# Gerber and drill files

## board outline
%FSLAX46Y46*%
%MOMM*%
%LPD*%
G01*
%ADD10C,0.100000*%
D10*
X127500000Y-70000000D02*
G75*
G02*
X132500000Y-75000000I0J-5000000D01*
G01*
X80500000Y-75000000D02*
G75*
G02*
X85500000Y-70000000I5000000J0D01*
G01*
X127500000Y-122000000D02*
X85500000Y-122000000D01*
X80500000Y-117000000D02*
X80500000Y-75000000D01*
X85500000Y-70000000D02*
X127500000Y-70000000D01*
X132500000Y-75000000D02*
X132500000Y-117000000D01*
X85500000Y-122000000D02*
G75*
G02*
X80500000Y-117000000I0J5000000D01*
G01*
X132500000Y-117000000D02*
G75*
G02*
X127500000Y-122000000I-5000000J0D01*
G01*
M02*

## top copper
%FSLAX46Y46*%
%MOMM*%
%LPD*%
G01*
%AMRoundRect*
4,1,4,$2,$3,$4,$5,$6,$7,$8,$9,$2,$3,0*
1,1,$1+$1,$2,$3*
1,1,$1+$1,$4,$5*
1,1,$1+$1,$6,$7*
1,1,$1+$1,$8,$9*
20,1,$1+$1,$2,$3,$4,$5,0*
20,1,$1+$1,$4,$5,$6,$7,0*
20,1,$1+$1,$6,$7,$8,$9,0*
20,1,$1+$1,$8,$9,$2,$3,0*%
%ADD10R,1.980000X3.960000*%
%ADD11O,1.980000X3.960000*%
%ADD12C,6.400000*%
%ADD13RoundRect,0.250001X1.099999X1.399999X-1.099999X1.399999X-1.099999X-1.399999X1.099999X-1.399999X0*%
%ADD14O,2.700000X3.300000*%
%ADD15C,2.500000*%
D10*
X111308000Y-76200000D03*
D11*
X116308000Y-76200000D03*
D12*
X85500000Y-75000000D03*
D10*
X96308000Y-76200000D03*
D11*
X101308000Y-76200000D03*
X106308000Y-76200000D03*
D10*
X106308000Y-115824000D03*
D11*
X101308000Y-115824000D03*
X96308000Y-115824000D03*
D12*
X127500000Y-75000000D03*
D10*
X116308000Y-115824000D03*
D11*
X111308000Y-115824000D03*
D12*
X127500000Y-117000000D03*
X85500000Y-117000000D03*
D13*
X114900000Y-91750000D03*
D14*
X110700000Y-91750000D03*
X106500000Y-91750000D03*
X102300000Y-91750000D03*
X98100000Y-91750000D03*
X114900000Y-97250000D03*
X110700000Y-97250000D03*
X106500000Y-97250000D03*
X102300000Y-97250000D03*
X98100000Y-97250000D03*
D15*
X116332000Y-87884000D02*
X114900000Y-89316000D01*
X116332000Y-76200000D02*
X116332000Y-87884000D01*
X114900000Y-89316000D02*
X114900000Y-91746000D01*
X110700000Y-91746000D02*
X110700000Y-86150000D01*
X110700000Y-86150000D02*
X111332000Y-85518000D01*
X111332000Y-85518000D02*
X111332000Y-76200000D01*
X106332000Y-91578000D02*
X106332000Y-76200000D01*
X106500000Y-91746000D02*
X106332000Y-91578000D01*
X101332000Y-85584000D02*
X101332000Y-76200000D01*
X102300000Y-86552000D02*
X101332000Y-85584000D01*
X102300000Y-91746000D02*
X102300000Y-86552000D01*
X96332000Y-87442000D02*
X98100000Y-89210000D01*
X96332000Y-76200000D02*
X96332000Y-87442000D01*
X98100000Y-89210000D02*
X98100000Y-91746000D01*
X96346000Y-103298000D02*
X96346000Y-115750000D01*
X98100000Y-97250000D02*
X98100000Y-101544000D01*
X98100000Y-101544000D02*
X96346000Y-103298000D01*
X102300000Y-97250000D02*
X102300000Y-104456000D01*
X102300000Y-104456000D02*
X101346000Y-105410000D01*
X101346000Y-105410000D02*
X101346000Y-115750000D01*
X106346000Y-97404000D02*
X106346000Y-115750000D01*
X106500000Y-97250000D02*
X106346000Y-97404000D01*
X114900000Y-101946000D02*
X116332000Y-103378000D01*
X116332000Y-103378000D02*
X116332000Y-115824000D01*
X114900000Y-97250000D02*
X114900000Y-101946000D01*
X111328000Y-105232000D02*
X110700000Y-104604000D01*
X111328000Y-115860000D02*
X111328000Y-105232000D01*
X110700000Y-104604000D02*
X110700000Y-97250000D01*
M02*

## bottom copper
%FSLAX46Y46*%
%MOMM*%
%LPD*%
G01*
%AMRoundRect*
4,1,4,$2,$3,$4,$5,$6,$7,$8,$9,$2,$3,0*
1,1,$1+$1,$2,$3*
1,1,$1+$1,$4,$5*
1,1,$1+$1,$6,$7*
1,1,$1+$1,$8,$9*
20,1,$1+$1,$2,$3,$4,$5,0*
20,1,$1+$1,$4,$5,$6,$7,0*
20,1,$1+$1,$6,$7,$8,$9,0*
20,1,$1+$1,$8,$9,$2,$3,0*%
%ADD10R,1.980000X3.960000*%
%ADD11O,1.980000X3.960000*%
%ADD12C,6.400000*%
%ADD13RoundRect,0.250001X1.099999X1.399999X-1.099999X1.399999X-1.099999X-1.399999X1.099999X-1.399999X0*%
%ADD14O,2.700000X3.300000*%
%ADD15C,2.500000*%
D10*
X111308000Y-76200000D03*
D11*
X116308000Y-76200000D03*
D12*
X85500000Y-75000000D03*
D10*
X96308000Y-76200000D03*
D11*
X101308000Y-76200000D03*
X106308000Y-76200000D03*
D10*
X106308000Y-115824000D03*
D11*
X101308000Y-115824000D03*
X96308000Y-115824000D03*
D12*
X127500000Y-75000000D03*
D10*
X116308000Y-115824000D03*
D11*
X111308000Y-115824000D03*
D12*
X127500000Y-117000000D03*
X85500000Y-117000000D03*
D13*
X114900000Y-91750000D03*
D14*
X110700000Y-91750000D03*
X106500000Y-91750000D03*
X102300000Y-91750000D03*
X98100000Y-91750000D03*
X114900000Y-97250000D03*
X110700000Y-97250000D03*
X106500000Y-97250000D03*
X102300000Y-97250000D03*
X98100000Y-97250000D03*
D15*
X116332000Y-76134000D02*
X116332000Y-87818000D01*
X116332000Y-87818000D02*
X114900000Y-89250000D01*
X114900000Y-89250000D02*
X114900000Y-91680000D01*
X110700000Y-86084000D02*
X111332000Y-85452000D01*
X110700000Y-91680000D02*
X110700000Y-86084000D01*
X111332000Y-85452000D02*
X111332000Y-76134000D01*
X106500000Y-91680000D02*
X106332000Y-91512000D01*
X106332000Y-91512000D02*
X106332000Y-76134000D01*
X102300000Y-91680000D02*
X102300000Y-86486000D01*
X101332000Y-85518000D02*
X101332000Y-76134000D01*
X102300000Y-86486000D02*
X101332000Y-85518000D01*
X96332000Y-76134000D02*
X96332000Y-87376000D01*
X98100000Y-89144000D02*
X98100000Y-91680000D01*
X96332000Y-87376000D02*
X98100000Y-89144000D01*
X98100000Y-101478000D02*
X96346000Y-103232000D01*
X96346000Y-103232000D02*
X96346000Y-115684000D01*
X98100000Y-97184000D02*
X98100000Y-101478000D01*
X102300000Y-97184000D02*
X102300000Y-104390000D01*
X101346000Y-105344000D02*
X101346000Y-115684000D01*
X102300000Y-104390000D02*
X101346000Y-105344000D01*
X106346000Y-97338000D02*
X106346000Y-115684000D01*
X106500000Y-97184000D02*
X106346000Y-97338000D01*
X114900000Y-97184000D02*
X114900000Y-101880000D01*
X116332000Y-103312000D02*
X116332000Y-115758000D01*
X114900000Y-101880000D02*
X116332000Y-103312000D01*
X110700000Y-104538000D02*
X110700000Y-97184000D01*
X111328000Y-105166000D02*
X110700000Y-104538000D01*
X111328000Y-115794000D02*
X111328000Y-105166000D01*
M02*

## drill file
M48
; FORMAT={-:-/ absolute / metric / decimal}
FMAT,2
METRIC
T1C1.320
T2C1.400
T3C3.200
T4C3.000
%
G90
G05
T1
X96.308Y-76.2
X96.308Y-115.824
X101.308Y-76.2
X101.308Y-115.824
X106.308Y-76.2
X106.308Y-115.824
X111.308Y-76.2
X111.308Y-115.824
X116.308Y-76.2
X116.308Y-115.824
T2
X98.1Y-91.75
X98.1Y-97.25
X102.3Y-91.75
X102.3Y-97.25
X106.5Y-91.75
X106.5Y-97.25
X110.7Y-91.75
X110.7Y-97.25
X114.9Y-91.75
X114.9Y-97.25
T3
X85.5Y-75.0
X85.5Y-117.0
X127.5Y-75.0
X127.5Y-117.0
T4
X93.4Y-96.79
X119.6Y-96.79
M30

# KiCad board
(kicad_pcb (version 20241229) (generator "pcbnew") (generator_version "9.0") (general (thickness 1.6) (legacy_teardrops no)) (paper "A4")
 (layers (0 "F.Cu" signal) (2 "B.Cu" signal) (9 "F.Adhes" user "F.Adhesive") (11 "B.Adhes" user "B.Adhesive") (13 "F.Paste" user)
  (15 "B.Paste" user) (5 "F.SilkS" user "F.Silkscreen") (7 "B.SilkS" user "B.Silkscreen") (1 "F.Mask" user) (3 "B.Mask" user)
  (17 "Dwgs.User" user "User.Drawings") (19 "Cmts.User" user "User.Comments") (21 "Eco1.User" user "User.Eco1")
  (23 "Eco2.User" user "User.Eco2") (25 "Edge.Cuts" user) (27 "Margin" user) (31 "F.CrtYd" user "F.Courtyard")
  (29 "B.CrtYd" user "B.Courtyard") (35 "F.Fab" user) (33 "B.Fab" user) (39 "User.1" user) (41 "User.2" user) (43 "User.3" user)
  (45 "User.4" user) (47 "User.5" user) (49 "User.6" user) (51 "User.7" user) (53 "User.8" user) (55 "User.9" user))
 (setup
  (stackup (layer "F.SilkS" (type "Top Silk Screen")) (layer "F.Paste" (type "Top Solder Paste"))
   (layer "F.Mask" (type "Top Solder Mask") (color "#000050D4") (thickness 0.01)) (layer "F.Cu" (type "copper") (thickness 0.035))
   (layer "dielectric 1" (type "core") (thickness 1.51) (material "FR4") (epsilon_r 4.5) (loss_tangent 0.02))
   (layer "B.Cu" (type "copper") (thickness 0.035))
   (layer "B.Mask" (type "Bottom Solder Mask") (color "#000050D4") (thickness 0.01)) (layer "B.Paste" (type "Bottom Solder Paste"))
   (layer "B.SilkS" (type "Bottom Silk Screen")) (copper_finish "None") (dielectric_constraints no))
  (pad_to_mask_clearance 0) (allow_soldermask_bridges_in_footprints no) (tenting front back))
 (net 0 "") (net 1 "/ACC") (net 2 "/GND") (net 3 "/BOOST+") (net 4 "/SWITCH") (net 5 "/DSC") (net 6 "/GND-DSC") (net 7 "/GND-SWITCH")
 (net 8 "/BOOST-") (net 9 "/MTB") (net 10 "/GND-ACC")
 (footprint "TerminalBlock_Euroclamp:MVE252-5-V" (layer "F.Cu") (at 113.808 76.2)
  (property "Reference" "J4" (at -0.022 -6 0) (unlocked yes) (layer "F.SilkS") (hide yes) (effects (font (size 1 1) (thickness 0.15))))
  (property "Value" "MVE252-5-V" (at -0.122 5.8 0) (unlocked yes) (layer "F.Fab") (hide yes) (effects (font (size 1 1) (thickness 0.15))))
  (pad "1" thru_hole rect (at -2.5 0) (size 1.98 3.96) (drill 1.32) (layers "*.Cu" "*.Mask") (remove_unused_layers no) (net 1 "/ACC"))
  (pad "2" thru_hole oval (at 2.5 0) (size 1.98 3.96) (drill 1.32) (layers "*.Cu" "*.Mask") (remove_unused_layers no) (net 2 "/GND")))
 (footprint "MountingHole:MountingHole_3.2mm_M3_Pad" (layer "F.Cu") (at 85.5 75)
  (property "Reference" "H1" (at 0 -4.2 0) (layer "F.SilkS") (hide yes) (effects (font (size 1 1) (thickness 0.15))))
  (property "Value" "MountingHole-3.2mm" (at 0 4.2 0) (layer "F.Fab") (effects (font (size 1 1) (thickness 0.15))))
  (pad "1" thru_hole circle (at 0 0) (size 6.4 6.4) (drill 3.2) (layers "*.Cu" "*.Mask") (remove_unused_layers no)))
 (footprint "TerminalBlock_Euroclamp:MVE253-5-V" (layer "F.Cu") (at 101.308 76.2)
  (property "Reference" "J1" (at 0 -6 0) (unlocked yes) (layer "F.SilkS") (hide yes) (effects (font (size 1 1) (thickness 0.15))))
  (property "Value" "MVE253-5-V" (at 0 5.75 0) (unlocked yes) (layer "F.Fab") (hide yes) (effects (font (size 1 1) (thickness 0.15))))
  (pad "1" thru_hole rect (at -5 0) (size 1.98 3.96) (drill 1.32) (layers "*.Cu" "*.Mask") (remove_unused_layers no) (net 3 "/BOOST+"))
  (pad "2" thru_hole oval (at 0 0) (size 1.98 3.96) (drill 1.32) (layers "*.Cu" "*.Mask") (remove_unused_layers no) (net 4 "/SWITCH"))
  (pad "3" thru_hole oval (at 5 0) (size 1.98 3.96) (drill 1.32) (layers "*.Cu" "*.Mask") (remove_unused_layers no) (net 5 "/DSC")))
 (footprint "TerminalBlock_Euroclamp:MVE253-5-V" (layer "F.Cu") (at 101.308 115.824 180)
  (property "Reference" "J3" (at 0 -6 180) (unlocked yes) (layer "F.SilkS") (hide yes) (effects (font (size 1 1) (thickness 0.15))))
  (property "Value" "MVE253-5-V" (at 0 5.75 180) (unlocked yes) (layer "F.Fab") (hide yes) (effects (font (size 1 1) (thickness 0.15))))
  (pad "1" thru_hole rect (at -5 0 180) (size 1.98 3.96) (drill 1.32) (layers "*.Cu" "*.Mask") (remove_unused_layers no) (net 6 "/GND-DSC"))
  (pad "2" thru_hole oval (at 0 0 180) (size 1.98 3.96) (drill 1.32) (layers "*.Cu" "*.Mask") (remove_unused_layers no)
   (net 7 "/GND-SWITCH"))
  (pad "3" thru_hole oval (at 5 0 180) (size 1.98 3.96) (drill 1.32) (layers "*.Cu" "*.Mask") (remove_unused_layers no) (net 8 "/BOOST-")))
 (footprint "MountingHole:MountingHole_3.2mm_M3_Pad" (layer "F.Cu") (at 127.5 75)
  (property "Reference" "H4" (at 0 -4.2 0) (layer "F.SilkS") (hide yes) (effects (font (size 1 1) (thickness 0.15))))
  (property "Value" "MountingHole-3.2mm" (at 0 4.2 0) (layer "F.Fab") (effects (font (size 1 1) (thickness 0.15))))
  (pad "1" thru_hole circle (at 0 0) (size 6.4 6.4) (drill 3.2) (layers "*.Cu" "*.Mask") (remove_unused_layers no)))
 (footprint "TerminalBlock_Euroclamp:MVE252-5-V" (layer "F.Cu") (at 113.808 115.824 180)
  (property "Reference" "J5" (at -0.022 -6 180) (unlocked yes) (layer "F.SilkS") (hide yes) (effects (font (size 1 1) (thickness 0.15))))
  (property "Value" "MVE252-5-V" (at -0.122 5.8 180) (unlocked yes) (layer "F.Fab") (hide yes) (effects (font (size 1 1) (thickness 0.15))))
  (pad "1" thru_hole rect (at -2.5 0 180) (size 1.98 3.96) (drill 1.32) (layers "*.Cu" "*.Mask") (remove_unused_layers no) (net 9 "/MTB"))
  (pad "2" thru_hole oval (at 2.5 0 180) (size 1.98 3.96) (drill 1.32) (layers "*.Cu" "*.Mask") (remove_unused_layers no)
   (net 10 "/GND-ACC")))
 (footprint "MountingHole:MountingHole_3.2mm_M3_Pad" (layer "F.Cu") (at 127.5 117)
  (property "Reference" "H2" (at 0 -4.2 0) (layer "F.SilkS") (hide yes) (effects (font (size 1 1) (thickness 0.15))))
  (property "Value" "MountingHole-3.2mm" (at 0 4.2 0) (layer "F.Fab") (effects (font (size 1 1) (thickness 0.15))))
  (pad "1" thru_hole circle (at 0 0) (size 6.4 6.4) (drill 3.2) (layers "*.Cu" "*.Mask") (remove_unused_layers no)))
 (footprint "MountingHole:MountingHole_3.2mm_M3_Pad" (layer "F.Cu") (at 85.5 117)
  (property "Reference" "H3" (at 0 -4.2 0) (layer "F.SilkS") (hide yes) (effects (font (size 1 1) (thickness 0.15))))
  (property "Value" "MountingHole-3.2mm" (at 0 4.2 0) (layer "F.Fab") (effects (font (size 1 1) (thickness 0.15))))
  (pad "1" thru_hole circle (at 0 0) (size 6.4 6.4) (drill 3.2) (layers "*.Cu" "*.Mask") (remove_unused_layers no)))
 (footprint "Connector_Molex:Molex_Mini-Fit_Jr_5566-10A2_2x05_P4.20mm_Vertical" (layer "B.Cu") (at 114.9 91.75 180)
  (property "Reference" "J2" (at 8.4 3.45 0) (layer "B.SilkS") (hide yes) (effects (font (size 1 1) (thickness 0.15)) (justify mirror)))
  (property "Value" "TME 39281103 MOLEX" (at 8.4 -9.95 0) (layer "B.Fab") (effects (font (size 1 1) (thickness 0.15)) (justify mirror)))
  (pad "" np_thru_hole circle (at -4.7 -5.04 180) (size 3 3) (drill 3) (layers "*.Cu" "*.Mask"))
  (pad "" np_thru_hole circle (at 21.5 -5.04 180) (size 3 3) (drill 3) (layers "*.Cu" "*.Mask"))
  (pad "1" thru_hole roundrect (at 0 0 180) (size 2.7 3.3) (drill 1.4) (layers "*.Cu" "*.Mask") (remove_unused_layers no)
   (roundrect_rratio 0.092593) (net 2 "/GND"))
  (pad "2" thru_hole oval (at 4.2 0 180) (size 2.7 3.3) (drill 1.4) (layers "*.Cu" "*.Mask") (remove_unused_layers no) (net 1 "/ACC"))
  (pad "3" thru_hole oval (at 8.4 0 180) (size 2.7 3.3) (drill 1.4) (layers "*.Cu" "*.Mask") (remove_unused_layers no) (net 5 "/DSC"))
  (pad "4" thru_hole oval (at 12.6 0 180) (size 2.7 3.3) (drill 1.4) (layers "*.Cu" "*.Mask") (remove_unused_layers no) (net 4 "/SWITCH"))
  (pad "5" thru_hole oval (at 16.8 0 180) (size 2.7 3.3) (drill 1.4) (layers "*.Cu" "*.Mask") (remove_unused_layers no) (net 3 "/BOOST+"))
  (pad "6" thru_hole oval (at 0 -5.5 180) (size 2.7 3.3) (drill 1.4) (layers "*.Cu" "*.Mask") (remove_unused_layers no) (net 9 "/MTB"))
  (pad "7" thru_hole oval (at 4.2 -5.5 180) (size 2.7 3.3) (drill 1.4) (layers "*.Cu" "*.Mask") (remove_unused_layers no)
   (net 10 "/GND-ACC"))
  (pad "8" thru_hole oval (at 8.4 -5.5 180) (size 2.7 3.3) (drill 1.4) (layers "*.Cu" "*.Mask") (remove_unused_layers no) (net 6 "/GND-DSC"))
  (pad "9" thru_hole oval (at 12.6 -5.5 180) (size 2.7 3.3) (drill 1.4) (layers "*.Cu" "*.Mask") (remove_unused_layers no)
   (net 7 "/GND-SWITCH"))
  (pad "10" thru_hole oval (at 16.8 -5.5 180) (size 2.7 3.3) (drill 1.4) (layers "*.Cu" "*.Mask") (remove_unused_layers no)
   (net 8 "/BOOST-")))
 (gr_arc (start 127.5 70) (mid 131.035534 71.464466) (end 132.5 75) (stroke (width 0.1) (type solid)) (layer "Edge.Cuts"))
 (gr_arc (start 80.5 75) (mid 81.964466 71.464466) (end 85.5 70) (stroke (width 0.1) (type solid)) (layer "Edge.Cuts"))
 (gr_line (start 127.5 122) (end 85.5 122) (stroke (width 0.1) (type solid)) (layer "Edge.Cuts"))
 (gr_line (start 80.5 117) (end 80.5 75) (stroke (width 0.1) (type solid)) (layer "Edge.Cuts"))
 (gr_line (start 85.5 70) (end 127.5 70) (stroke (width 0.1) (type solid)) (layer "Edge.Cuts"))
 (gr_line (start 132.5 75) (end 132.5 117) (stroke (width 0.1) (type solid)) (layer "Edge.Cuts"))
 (gr_arc (start 85.5 122) (mid 81.964466 120.535534) (end 80.5 117) (stroke (width 0.1) (type solid)) (layer "Edge.Cuts"))
 (gr_arc (start 132.5 117) (mid 131.035534 120.535534) (end 127.5 122) (stroke (width 0.1) (type solid)) (layer "Edge.Cuts"))
 (segment (start 116.332 87.884) (end 114.9 89.316) (width 2.5) (layer "F.Cu") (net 2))
 (segment (start 116.332 76.2) (end 116.332 87.884) (width 2.5) (layer "F.Cu") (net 2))
 (segment (start 114.9 89.316) (end 114.9 91.746) (width 2.5) (layer "F.Cu") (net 2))
 (segment (start 116.332 76.134) (end 116.332 87.818) (width 2.5) (layer "B.Cu") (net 2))
 (segment (start 116.332 87.818) (end 114.9 89.25) (width 2.5) (layer "B.Cu") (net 2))
 (segment (start 114.9 89.25) (end 114.9 91.68) (width 2.5) (layer "B.Cu") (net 2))
 (segment (start 110.7 91.746) (end 110.7 86.15) (width 2.5) (layer "F.Cu") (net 1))
 (segment (start 110.7 86.15) (end 111.332 85.518) (width 2.5) (layer "F.Cu") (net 1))
 (segment (start 111.332 85.518) (end 111.332 76.2) (width 2.5) (layer "F.Cu") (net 1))
 (segment (start 110.7 86.084) (end 111.332 85.452) (width 2.5) (layer "B.Cu") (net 1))
 (segment (start 110.7 91.68) (end 110.7 86.084) (width 2.5) (layer "B.Cu") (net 1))
 (segment (start 111.332 85.452) (end 111.332 76.134) (width 2.5) (layer "B.Cu") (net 1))
 (segment (start 106.332 91.578) (end 106.332 76.2) (width 2.5) (layer "F.Cu") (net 5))
 (segment (start 106.5 91.746) (end 106.332 91.578) (width 2.5) (layer "F.Cu") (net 5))
 (segment (start 106.5 91.68) (end 106.332 91.512) (width 2.5) (layer "B.Cu") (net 5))
 (segment (start 106.332 91.512) (end 106.332 76.134) (width 2.5) (layer "B.Cu") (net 5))
 (segment (start 101.332 85.584) (end 101.332 76.2) (width 2.5) (layer "F.Cu") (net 4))
 (segment (start 102.3 86.552) (end 101.332 85.584) (width 2.5) (layer "F.Cu") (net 4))
 (segment (start 102.3 91.746) (end 102.3 86.552) (width 2.5) (layer "F.Cu") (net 4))
 (segment (start 102.3 91.68) (end 102.3 86.486) (width 2.5) (layer "B.Cu") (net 4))
 (segment (start 101.332 85.518) (end 101.332 76.134) (width 2.5) (layer "B.Cu") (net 4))
 (segment (start 102.3 86.486) (end 101.332 85.518) (width 2.5) (layer "B.Cu") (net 4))
 (segment (start 96.332 87.442) (end 98.1 89.21) (width 2.5) (layer "F.Cu") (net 3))
 (segment (start 96.332 76.2) (end 96.332 87.442) (width 2.5) (layer "F.Cu") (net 3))
 (segment (start 98.1 89.21) (end 98.1 91.746) (width 2.5) (layer "F.Cu") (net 3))
 (segment (start 96.332 76.134) (end 96.332 87.376) (width 2.5) (layer "B.Cu") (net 3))
 (segment (start 98.1 89.144) (end 98.1 91.68) (width 2.5) (layer "B.Cu") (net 3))
 (segment (start 96.332 87.376) (end 98.1 89.144) (width 2.5) (layer "B.Cu") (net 3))
 (segment (start 96.346 103.298) (end 96.346 115.75) (width 2.5) (layer "F.Cu") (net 8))
 (segment (start 98.1 97.25) (end 98.1 101.544) (width 2.5) (layer "F.Cu") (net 8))
 (segment (start 98.1 101.544) (end 96.346 103.298) (width 2.5) (layer "F.Cu") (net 8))
 (segment (start 98.1 101.478) (end 96.346 103.232) (width 2.5) (layer "B.Cu") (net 8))
 (segment (start 96.346 103.232) (end 96.346 115.684) (width 2.5) (layer "B.Cu") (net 8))
 (segment (start 98.1 97.184) (end 98.1 101.478) (width 2.5) (layer "B.Cu") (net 8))
 (segment (start 102.3 97.25) (end 102.3 104.456) (width 2.5) (layer "F.Cu") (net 7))
 (segment (start 102.3 104.456) (end 101.346 105.41) (width 2.5) (layer "F.Cu") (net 7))
 (segment (start 101.346 105.41) (end 101.346 115.75) (width 2.5) (layer "F.Cu") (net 7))
 (segment (start 102.3 97.184) (end 102.3 104.39) (width 2.5) (layer "B.Cu") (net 7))
 (segment (start 101.346 105.344) (end 101.346 115.684) (width 2.5) (layer "B.Cu") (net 7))
 (segment (start 102.3 104.39) (end 101.346 105.344) (width 2.5) (layer "B.Cu") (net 7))
 (segment (start 106.346 97.404) (end 106.346 115.75) (width 2.5) (layer "F.Cu") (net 6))
 (segment (start 106.5 97.25) (end 106.346 97.404) (width 2.5) (layer "F.Cu") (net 6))
 (segment (start 106.346 97.338) (end 106.346 115.684) (width 2.5) (layer "B.Cu") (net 6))
 (segment (start 106.5 97.184) (end 106.346 97.338) (width 2.5) (layer "B.Cu") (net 6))
 (segment (start 114.9 101.946) (end 116.332 103.378) (width 2.5) (layer "F.Cu") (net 9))
 (segment (start 116.332 103.378) (end 116.332 115.824) (width 2.5) (layer "F.Cu") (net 9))
 (segment (start 114.9 97.25) (end 114.9 101.946) (width 2.5) (layer "F.Cu") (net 9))
 (segment (start 114.9 97.184) (end 114.9 101.88) (width 2.5) (layer "B.Cu") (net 9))
 (segment (start 116.332 103.312) (end 116.332 115.758) (width 2.5) (layer "B.Cu") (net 9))
 (segment (start 114.9 101.88) (end 116.332 103.312) (width 2.5) (layer "B.Cu") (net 9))
 (segment (start 111.328 105.232) (end 110.7 104.604) (width 2.5) (layer "F.Cu") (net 10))
 (segment (start 111.328 115.86) (end 111.328 105.232) (width 2.5) (layer "F.Cu") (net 10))
 (segment (start 110.7 104.604) (end 110.7 97.25) (width 2.5) (layer "F.Cu") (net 10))
 (segment (start 110.7 104.538) (end 110.7 97.184) (width 2.5) (layer "B.Cu") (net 10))
 (segment (start 111.328 105.166) (end 110.7 104.538) (width 2.5) (layer "B.Cu") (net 10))
 (segment (start 111.328 115.794) (end 111.328 105.166) (width 2.5) (layer "B.Cu") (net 10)))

